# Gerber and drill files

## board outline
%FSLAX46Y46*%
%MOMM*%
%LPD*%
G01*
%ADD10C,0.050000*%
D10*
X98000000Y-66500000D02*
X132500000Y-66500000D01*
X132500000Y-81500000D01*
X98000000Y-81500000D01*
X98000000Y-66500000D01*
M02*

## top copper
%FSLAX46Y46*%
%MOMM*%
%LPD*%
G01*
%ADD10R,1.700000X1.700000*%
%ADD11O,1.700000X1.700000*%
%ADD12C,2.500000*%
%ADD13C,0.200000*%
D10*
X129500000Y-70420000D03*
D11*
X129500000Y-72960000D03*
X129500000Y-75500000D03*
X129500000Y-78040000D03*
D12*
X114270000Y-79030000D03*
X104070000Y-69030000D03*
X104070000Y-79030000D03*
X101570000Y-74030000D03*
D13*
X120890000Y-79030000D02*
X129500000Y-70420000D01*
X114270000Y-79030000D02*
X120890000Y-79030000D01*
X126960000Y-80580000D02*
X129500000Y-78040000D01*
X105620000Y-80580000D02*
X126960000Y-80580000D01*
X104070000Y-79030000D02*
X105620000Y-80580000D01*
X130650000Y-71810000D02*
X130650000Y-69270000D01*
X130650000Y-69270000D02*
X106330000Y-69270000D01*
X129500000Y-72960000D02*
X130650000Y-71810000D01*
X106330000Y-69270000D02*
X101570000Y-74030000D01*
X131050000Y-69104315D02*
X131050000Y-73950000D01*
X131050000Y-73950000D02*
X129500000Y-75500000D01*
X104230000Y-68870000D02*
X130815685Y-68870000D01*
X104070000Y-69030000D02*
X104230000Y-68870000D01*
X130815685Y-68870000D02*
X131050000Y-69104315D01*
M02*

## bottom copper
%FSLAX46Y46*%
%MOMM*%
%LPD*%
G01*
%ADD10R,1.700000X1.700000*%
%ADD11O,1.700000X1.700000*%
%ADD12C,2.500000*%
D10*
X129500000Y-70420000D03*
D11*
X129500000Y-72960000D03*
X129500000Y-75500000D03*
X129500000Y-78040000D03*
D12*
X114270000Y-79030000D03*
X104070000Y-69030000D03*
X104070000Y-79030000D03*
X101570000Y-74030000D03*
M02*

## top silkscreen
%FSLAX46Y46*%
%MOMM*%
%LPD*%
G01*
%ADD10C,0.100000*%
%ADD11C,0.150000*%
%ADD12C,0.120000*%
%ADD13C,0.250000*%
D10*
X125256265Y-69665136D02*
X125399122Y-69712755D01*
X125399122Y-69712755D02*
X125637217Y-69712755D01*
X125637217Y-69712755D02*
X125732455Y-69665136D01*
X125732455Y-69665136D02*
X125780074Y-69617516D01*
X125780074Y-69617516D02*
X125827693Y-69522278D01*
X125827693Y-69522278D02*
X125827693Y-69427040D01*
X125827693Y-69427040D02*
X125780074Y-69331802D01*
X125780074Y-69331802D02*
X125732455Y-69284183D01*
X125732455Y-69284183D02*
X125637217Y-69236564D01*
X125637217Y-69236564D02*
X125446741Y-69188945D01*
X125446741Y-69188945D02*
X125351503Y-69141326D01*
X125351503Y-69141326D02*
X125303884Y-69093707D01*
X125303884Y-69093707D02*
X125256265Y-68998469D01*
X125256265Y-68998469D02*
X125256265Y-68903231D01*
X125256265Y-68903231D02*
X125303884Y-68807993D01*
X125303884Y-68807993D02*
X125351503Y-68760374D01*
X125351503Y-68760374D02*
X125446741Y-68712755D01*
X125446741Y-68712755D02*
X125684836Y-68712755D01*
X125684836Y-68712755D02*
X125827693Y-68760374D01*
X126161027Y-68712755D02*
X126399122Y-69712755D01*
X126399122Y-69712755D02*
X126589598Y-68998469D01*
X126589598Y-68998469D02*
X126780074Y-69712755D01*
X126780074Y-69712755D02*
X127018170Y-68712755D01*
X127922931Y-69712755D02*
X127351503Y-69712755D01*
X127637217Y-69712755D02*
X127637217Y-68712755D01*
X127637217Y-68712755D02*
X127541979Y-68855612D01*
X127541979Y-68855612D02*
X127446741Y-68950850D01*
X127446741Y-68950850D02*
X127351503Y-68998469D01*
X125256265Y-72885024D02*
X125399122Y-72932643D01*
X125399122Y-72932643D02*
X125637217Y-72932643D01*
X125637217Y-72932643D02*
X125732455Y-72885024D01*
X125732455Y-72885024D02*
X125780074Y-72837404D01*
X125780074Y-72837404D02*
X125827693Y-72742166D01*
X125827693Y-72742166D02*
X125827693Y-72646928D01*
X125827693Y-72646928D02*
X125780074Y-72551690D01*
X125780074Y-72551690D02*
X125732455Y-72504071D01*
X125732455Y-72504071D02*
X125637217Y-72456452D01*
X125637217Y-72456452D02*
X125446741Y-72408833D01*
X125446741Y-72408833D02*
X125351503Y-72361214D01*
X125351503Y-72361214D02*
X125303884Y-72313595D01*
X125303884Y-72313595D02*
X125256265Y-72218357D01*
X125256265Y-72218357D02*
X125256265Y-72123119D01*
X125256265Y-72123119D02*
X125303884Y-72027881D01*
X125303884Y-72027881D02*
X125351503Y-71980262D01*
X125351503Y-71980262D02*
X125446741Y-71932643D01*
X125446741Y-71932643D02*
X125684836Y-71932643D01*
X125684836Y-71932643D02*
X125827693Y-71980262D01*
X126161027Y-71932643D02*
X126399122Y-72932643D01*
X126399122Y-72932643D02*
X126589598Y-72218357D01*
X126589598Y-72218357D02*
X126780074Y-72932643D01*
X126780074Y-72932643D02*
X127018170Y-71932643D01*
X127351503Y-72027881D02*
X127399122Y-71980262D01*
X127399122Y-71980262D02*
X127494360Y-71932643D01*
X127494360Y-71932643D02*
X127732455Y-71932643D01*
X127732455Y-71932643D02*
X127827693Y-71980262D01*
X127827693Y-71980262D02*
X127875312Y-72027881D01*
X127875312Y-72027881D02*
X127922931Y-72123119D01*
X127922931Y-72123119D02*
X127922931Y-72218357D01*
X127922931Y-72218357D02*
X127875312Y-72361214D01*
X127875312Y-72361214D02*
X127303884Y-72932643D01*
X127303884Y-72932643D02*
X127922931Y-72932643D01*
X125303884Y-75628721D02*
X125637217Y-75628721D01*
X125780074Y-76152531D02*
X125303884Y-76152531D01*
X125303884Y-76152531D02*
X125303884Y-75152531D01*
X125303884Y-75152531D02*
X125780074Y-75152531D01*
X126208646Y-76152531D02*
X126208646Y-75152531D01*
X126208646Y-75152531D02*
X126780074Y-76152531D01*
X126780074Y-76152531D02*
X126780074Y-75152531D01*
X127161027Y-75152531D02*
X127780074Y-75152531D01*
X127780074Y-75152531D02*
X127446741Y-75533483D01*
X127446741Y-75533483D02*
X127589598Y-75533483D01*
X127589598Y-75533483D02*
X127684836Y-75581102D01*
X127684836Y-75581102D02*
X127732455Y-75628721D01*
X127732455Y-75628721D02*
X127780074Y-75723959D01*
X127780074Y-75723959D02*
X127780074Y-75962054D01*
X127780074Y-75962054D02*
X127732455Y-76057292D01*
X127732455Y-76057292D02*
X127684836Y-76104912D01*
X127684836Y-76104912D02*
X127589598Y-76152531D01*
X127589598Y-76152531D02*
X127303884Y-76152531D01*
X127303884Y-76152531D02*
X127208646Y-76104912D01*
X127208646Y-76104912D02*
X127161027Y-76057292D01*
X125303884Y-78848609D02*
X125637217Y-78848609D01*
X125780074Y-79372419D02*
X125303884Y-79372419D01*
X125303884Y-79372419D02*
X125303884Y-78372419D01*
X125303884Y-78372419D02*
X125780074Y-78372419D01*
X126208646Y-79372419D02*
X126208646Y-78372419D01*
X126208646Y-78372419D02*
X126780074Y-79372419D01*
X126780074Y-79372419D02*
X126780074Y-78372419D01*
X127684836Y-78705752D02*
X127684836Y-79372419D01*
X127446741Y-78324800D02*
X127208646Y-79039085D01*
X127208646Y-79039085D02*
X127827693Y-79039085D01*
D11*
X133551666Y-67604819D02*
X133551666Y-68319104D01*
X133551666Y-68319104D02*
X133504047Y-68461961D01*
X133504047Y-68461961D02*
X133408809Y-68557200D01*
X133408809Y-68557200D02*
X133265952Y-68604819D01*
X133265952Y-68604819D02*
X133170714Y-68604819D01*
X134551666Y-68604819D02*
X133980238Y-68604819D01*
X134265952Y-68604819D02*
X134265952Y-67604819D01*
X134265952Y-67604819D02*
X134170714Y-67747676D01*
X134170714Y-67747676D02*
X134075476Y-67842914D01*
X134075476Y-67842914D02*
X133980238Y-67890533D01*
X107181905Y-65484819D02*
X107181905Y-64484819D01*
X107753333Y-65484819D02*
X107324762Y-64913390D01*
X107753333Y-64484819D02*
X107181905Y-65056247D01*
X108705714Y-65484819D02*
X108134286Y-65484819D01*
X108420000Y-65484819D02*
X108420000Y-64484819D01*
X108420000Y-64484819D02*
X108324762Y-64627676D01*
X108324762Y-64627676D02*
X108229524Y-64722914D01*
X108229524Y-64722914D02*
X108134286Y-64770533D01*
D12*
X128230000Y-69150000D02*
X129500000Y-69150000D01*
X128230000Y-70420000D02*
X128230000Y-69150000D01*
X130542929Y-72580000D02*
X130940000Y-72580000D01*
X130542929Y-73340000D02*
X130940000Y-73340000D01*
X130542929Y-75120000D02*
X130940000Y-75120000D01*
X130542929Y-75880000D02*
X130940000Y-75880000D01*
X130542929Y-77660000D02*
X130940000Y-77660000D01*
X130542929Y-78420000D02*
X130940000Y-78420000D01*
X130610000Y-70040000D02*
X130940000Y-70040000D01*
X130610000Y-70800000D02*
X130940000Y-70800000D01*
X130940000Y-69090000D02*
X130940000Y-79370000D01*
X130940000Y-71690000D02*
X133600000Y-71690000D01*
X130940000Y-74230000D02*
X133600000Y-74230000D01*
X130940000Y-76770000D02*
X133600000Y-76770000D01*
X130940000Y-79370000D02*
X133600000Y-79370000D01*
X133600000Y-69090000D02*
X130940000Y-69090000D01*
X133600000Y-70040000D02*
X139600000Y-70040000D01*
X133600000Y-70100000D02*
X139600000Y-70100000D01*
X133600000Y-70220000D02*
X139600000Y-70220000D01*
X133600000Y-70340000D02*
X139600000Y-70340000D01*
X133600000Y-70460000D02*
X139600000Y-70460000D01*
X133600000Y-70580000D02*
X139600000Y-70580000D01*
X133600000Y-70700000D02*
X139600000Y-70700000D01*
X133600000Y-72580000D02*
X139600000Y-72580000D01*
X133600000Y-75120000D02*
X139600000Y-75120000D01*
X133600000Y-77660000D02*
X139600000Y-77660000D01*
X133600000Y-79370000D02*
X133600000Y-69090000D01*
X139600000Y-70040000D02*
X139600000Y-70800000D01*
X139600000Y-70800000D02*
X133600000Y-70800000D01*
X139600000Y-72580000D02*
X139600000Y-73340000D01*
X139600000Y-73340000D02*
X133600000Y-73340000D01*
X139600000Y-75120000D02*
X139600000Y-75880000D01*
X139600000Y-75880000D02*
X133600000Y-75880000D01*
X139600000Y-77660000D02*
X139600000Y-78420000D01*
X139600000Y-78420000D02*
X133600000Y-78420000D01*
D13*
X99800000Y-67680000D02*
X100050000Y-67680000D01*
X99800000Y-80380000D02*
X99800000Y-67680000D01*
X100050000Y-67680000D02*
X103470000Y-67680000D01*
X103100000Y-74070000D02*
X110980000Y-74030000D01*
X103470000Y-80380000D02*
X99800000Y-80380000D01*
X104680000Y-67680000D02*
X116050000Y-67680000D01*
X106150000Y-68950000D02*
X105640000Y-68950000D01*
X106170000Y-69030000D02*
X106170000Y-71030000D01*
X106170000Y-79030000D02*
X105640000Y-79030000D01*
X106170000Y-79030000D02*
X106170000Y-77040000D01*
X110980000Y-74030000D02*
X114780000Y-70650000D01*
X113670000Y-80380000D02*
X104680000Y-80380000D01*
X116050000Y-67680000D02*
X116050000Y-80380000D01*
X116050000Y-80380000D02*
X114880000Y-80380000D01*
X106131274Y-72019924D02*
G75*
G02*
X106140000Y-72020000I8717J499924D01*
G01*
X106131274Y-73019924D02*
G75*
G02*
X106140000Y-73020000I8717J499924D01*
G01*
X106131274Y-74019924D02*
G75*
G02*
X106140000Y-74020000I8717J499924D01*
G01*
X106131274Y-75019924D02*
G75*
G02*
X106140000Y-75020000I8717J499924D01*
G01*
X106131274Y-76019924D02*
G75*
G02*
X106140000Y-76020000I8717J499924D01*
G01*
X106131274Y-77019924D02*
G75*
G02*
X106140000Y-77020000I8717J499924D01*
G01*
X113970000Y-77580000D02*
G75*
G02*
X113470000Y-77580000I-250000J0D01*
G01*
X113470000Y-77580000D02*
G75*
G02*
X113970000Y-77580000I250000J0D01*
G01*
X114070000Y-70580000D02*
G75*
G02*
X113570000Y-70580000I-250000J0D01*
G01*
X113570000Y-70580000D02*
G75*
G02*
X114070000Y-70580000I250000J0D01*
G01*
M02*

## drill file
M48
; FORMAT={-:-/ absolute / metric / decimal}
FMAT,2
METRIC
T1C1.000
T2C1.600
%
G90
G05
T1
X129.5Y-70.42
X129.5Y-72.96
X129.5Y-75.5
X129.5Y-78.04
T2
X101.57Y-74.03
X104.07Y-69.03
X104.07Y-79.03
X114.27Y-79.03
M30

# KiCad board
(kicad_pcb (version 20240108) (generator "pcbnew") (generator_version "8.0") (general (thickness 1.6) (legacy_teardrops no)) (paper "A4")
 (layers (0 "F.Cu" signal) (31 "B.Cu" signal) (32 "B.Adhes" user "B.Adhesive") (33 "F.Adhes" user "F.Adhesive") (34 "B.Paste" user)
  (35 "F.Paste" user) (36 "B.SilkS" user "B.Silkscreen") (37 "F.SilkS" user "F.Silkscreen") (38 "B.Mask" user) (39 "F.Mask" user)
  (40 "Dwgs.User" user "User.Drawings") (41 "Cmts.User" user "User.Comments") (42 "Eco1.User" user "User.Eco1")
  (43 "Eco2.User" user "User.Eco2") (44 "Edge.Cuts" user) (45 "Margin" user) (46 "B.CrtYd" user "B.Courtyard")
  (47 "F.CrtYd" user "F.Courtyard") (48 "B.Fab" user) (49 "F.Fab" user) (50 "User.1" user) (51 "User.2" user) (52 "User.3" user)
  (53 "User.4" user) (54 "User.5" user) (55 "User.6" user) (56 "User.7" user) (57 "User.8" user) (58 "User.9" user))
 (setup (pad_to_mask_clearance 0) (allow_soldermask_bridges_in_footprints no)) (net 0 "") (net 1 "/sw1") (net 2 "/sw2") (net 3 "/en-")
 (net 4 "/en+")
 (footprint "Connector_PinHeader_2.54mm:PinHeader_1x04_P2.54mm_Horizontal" (layer "F.Cu") (at 129.5 70.42)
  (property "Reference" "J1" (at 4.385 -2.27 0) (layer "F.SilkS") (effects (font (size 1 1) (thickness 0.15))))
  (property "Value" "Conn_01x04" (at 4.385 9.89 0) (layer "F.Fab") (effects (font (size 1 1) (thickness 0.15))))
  (fp_line (start -1.27 -1.27) (end 0 -1.27) (stroke (width 0.12) (type solid)) (layer "F.SilkS"))
  (fp_line (start -1.27 0) (end -1.27 -1.27) (stroke (width 0.12) (type solid)) (layer "F.SilkS"))
  (fp_line (start 1.042929 2.16) (end 1.44 2.16) (stroke (width 0.12) (type solid)) (layer "F.SilkS"))
  (fp_line (start 1.042929 2.92) (end 1.44 2.92) (stroke (width 0.12) (type solid)) (layer "F.SilkS"))
  (fp_line (start 1.042929 4.7) (end 1.44 4.7) (stroke (width 0.12) (type solid)) (layer "F.SilkS"))
  (fp_line (start 1.042929 5.46) (end 1.44 5.46) (stroke (width 0.12) (type solid)) (layer "F.SilkS"))
  (fp_line (start 1.042929 7.24) (end 1.44 7.24) (stroke (width 0.12) (type solid)) (layer "F.SilkS"))
  (fp_line (start 1.042929 8) (end 1.44 8) (stroke (width 0.12) (type solid)) (layer "F.SilkS"))
  (fp_line (start 1.11 -0.38) (end 1.44 -0.38) (stroke (width 0.12) (type solid)) (layer "F.SilkS"))
  (fp_line (start 1.11 0.38) (end 1.44 0.38) (stroke (width 0.12) (type solid)) (layer "F.SilkS"))
  (fp_line (start 1.44 -1.33) (end 1.44 8.95) (stroke (width 0.12) (type solid)) (layer "F.SilkS"))
  (fp_line (start 1.44 1.27) (end 4.1 1.27) (stroke (width 0.12) (type solid)) (layer "F.SilkS"))
  (fp_line (start 1.44 3.81) (end 4.1 3.81) (stroke (width 0.12) (type solid)) (layer "F.SilkS"))
  (fp_line (start 1.44 6.35) (end 4.1 6.35) (stroke (width 0.12) (type solid)) (layer "F.SilkS"))
  (fp_line (start 1.44 8.95) (end 4.1 8.95) (stroke (width 0.12) (type solid)) (layer "F.SilkS"))
  (fp_line (start 4.1 -1.33) (end 1.44 -1.33) (stroke (width 0.12) (type solid)) (layer "F.SilkS"))
  (fp_line (start 4.1 -0.38) (end 10.1 -0.38) (stroke (width 0.12) (type solid)) (layer "F.SilkS"))
  (fp_line (start 4.1 -0.32) (end 10.1 -0.32) (stroke (width 0.12) (type solid)) (layer "F.SilkS"))
  (fp_line (start 4.1 -0.2) (end 10.1 -0.2) (stroke (width 0.12) (type solid)) (layer "F.SilkS"))
  (fp_line (start 4.1 -0.08) (end 10.1 -0.08) (stroke (width 0.12) (type solid)) (layer "F.SilkS"))
  (fp_line (start 4.1 0.04) (end 10.1 0.04) (stroke (width 0.12) (type solid)) (layer "F.SilkS"))
  (fp_line (start 4.1 0.16) (end 10.1 0.16) (stroke (width 0.12) (type solid)) (layer "F.SilkS"))
  (fp_line (start 4.1 0.28) (end 10.1 0.28) (stroke (width 0.12) (type solid)) (layer "F.SilkS"))
  (fp_line (start 4.1 2.16) (end 10.1 2.16) (stroke (width 0.12) (type solid)) (layer "F.SilkS"))
  (fp_line (start 4.1 4.7) (end 10.1 4.7) (stroke (width 0.12) (type solid)) (layer "F.SilkS"))
  (fp_line (start 4.1 7.24) (end 10.1 7.24) (stroke (width 0.12) (type solid)) (layer "F.SilkS"))
  (fp_line (start 4.1 8.95) (end 4.1 -1.33) (stroke (width 0.12) (type solid)) (layer "F.SilkS"))
  (fp_line (start 10.1 -0.38) (end 10.1 0.38) (stroke (width 0.12) (type solid)) (layer "F.SilkS"))
  (fp_line (start 10.1 0.38) (end 4.1 0.38) (stroke (width 0.12) (type solid)) (layer "F.SilkS"))
  (fp_line (start 10.1 2.16) (end 10.1 2.92) (stroke (width 0.12) (type solid)) (layer "F.SilkS"))
  (fp_line (start 10.1 2.92) (end 4.1 2.92) (stroke (width 0.12) (type solid)) (layer "F.SilkS"))
  (fp_line (start 10.1 4.7) (end 10.1 5.46) (stroke (width 0.12) (type solid)) (layer "F.SilkS"))
  (fp_line (start 10.1 5.46) (end 4.1 5.46) (stroke (width 0.12) (type solid)) (layer "F.SilkS"))
  (fp_line (start 10.1 7.24) (end 10.1 8) (stroke (width 0.12) (type solid)) (layer "F.SilkS"))
  (fp_line (start 10.1 8) (end 4.1 8) (stroke (width 0.12) (type solid)) (layer "F.SilkS"))
  (pad "1" thru_hole rect (at 0 0) (size 1.7 1.7) (drill 1) (layers "*.Cu" "*.Mask") (remove_unused_layers no) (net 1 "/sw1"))
  (pad "2" thru_hole oval (at 0 2.54) (size 1.7 1.7) (drill 1) (layers "*.Cu" "*.Mask") (remove_unused_layers no) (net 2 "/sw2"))
  (pad "3" thru_hole oval (at 0 5.08) (size 1.7 1.7) (drill 1) (layers "*.Cu" "*.Mask") (remove_unused_layers no) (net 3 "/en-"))
  (pad "4" thru_hole oval (at 0 7.62) (size 1.7 1.7) (drill 1) (layers "*.Cu" "*.Mask") (remove_unused_layers no) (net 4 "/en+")))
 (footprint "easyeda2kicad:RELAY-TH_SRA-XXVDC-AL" (layer "F.Cu") (at 107.92 74.03)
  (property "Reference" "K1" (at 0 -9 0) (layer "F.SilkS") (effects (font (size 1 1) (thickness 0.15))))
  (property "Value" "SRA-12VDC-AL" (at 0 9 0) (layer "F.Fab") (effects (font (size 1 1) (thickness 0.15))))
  (fp_line (start -8.12 -6.35) (end -7.87 -6.35) (stroke (width 0.25) (type solid)) (layer "F.SilkS"))
  (fp_line (start -8.12 6.35) (end -8.12 -6.35) (stroke (width 0.25) (type solid)) (layer "F.SilkS"))
  (fp_line (start -7.87 -6.35) (end -4.45 -6.35) (stroke (width 0.25) (type solid)) (layer "F.SilkS"))
  (fp_line (start -4.82 0.04) (end 3.06 0) (stroke (width 0.25) (type solid)) (layer "F.SilkS"))
  (fp_line (start -4.45 6.35) (end -8.12 6.35) (stroke (width 0.25) (type solid)) (layer "F.SilkS"))
  (fp_line (start -3.24 -6.35) (end 8.13 -6.35) (stroke (width 0.25) (type solid)) (layer "F.SilkS"))
  (fp_line (start -1.77 -5.08) (end -2.28 -5.08) (stroke (width 0.25) (type solid)) (layer "F.SilkS"))
  (fp_line (start -1.75 -5) (end -1.75 -3) (stroke (width 0.25) (type solid)) (layer "F.SilkS"))
  (fp_line (start -1.75 5) (end -2.28 5) (stroke (width 0.25) (type solid)) (layer "F.SilkS"))
  (fp_line (start -1.75 5) (end -1.75 3.01) (stroke (width 0.25) (type solid)) (layer "F.SilkS"))
  (fp_line (start 3.06 0) (end 6.86 -3.38) (stroke (width 0.25) (type solid)) (layer "F.SilkS"))
  (fp_line (start 5.75 6.35) (end -3.24 6.35) (stroke (width 0.25) (type solid)) (layer "F.SilkS"))
  (fp_line (start 8.13 -6.35) (end 8.13 6.35) (stroke (width 0.25) (type solid)) (layer "F.SilkS"))
  (fp_line (start 8.13 6.35) (end 6.96 6.35) (stroke (width 0.25) (type solid)) (layer "F.SilkS"))
  (fp_arc (start -1.788726 -2.010076) (mid -1.775637 -3.009981) (end -1.78 -2.01) (stroke (width 0.25) (type solid)) (layer "F.SilkS"))
  (fp_arc (start -1.788726 -1.010076) (mid -1.775637 -2.009981) (end -1.78 -1.01) (stroke (width 0.25) (type solid)) (layer "F.SilkS"))
  (fp_arc (start -1.788726 -0.010076) (mid -1.775637 -1.009981) (end -1.78 -0.01) (stroke (width 0.25) (type solid)) (layer "F.SilkS"))
  (fp_arc (start -1.788726 0.989924) (mid -1.775637 -0.009981) (end -1.78 0.99) (stroke (width 0.25) (type solid)) (layer "F.SilkS"))
  (fp_arc (start -1.788726 1.989924) (mid -1.775637 0.990019) (end -1.78 1.99) (stroke (width 0.25) (type solid)) (layer "F.SilkS"))
  (fp_arc (start -1.788726 2.989924) (mid -1.775637 1.990019) (end -1.78 2.99) (stroke (width 0.25) (type solid)) (layer "F.SilkS"))
  (fp_circle (center 5.8 3.55) (end 6.05 3.55) (stroke (width 0.25) (type solid)) (fill none) (layer "F.SilkS"))
  (fp_circle (center 5.9 -3.45) (end 6.15 -3.45) (stroke (width 0.25) (type solid)) (fill none) (layer "F.SilkS"))
  (pad "1" thru_hole circle (at 6.35 5) (size 2.5 2.5) (drill 1.599997) (layers "*.Cu" "*.Mask") (remove_unused_layers no) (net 1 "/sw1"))
  (pad "3" thru_hole circle (at -3.85 -5) (size 2.5 2.5) (drill 1.599997) (layers "*.Cu" "*.Mask") (remove_unused_layers no) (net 3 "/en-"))
  (pad "4" thru_hole circle (at -3.85 5) (size 2.5 2.5) (drill 1.599997) (layers "*.Cu" "*.Mask") (remove_unused_layers no) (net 4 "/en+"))
  (pad "5" thru_hole circle (at -6.35 0) (size 2.5 2.5) (drill 1.599997) (layers "*.Cu" "*.Mask") (remove_unused_layers no) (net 2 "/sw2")))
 (gr_rect (start 98 66.5) (end 132.5 81.5) (stroke (width 0.05) (type default)) (fill none) (layer "Edge.Cuts"))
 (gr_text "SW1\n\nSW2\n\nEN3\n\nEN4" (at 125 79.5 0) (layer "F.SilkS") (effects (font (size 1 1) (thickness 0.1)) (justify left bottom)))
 (segment (start 120.89 79.03) (end 129.5 70.42) (width 0.2) (layer "F.Cu") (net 1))
 (segment (start 114.27 79.03) (end 120.89 79.03) (width 0.2) (layer "F.Cu") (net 1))
 (segment (start 126.96 80.58) (end 129.5 78.04) (width 0.2) (layer "F.Cu") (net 4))
 (segment (start 105.62 80.58) (end 126.96 80.58) (width 0.2) (layer "F.Cu") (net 4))
 (segment (start 104.07 79.03) (end 105.62 80.58) (width 0.2) (layer "F.Cu") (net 4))
 (segment (start 130.65 71.81) (end 130.65 69.27) (width 0.2) (layer "F.Cu") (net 2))
 (segment (start 130.65 69.27) (end 106.33 69.27) (width 0.2) (layer "F.Cu") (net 2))
 (segment (start 129.5 72.96) (end 130.65 71.81) (width 0.2) (layer "F.Cu") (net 2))
 (segment (start 106.33 69.27) (end 101.57 74.03) (width 0.2) (layer "F.Cu") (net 2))
 (segment (start 131.05 69.104315) (end 131.05 73.95) (width 0.2) (layer "F.Cu") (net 3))
 (segment (start 131.05 73.95) (end 129.5 75.5) (width 0.2) (layer "F.Cu") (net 3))
 (segment (start 104.23 68.87) (end 130.815685 68.87) (width 0.2) (layer "F.Cu") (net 3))
 (segment (start 104.07 69.03) (end 104.23 68.87) (width 0.2) (layer "F.Cu") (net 3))
 (segment (start 130.815685 68.87) (end 131.05 69.104315) (width 0.2) (layer "F.Cu") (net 3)))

